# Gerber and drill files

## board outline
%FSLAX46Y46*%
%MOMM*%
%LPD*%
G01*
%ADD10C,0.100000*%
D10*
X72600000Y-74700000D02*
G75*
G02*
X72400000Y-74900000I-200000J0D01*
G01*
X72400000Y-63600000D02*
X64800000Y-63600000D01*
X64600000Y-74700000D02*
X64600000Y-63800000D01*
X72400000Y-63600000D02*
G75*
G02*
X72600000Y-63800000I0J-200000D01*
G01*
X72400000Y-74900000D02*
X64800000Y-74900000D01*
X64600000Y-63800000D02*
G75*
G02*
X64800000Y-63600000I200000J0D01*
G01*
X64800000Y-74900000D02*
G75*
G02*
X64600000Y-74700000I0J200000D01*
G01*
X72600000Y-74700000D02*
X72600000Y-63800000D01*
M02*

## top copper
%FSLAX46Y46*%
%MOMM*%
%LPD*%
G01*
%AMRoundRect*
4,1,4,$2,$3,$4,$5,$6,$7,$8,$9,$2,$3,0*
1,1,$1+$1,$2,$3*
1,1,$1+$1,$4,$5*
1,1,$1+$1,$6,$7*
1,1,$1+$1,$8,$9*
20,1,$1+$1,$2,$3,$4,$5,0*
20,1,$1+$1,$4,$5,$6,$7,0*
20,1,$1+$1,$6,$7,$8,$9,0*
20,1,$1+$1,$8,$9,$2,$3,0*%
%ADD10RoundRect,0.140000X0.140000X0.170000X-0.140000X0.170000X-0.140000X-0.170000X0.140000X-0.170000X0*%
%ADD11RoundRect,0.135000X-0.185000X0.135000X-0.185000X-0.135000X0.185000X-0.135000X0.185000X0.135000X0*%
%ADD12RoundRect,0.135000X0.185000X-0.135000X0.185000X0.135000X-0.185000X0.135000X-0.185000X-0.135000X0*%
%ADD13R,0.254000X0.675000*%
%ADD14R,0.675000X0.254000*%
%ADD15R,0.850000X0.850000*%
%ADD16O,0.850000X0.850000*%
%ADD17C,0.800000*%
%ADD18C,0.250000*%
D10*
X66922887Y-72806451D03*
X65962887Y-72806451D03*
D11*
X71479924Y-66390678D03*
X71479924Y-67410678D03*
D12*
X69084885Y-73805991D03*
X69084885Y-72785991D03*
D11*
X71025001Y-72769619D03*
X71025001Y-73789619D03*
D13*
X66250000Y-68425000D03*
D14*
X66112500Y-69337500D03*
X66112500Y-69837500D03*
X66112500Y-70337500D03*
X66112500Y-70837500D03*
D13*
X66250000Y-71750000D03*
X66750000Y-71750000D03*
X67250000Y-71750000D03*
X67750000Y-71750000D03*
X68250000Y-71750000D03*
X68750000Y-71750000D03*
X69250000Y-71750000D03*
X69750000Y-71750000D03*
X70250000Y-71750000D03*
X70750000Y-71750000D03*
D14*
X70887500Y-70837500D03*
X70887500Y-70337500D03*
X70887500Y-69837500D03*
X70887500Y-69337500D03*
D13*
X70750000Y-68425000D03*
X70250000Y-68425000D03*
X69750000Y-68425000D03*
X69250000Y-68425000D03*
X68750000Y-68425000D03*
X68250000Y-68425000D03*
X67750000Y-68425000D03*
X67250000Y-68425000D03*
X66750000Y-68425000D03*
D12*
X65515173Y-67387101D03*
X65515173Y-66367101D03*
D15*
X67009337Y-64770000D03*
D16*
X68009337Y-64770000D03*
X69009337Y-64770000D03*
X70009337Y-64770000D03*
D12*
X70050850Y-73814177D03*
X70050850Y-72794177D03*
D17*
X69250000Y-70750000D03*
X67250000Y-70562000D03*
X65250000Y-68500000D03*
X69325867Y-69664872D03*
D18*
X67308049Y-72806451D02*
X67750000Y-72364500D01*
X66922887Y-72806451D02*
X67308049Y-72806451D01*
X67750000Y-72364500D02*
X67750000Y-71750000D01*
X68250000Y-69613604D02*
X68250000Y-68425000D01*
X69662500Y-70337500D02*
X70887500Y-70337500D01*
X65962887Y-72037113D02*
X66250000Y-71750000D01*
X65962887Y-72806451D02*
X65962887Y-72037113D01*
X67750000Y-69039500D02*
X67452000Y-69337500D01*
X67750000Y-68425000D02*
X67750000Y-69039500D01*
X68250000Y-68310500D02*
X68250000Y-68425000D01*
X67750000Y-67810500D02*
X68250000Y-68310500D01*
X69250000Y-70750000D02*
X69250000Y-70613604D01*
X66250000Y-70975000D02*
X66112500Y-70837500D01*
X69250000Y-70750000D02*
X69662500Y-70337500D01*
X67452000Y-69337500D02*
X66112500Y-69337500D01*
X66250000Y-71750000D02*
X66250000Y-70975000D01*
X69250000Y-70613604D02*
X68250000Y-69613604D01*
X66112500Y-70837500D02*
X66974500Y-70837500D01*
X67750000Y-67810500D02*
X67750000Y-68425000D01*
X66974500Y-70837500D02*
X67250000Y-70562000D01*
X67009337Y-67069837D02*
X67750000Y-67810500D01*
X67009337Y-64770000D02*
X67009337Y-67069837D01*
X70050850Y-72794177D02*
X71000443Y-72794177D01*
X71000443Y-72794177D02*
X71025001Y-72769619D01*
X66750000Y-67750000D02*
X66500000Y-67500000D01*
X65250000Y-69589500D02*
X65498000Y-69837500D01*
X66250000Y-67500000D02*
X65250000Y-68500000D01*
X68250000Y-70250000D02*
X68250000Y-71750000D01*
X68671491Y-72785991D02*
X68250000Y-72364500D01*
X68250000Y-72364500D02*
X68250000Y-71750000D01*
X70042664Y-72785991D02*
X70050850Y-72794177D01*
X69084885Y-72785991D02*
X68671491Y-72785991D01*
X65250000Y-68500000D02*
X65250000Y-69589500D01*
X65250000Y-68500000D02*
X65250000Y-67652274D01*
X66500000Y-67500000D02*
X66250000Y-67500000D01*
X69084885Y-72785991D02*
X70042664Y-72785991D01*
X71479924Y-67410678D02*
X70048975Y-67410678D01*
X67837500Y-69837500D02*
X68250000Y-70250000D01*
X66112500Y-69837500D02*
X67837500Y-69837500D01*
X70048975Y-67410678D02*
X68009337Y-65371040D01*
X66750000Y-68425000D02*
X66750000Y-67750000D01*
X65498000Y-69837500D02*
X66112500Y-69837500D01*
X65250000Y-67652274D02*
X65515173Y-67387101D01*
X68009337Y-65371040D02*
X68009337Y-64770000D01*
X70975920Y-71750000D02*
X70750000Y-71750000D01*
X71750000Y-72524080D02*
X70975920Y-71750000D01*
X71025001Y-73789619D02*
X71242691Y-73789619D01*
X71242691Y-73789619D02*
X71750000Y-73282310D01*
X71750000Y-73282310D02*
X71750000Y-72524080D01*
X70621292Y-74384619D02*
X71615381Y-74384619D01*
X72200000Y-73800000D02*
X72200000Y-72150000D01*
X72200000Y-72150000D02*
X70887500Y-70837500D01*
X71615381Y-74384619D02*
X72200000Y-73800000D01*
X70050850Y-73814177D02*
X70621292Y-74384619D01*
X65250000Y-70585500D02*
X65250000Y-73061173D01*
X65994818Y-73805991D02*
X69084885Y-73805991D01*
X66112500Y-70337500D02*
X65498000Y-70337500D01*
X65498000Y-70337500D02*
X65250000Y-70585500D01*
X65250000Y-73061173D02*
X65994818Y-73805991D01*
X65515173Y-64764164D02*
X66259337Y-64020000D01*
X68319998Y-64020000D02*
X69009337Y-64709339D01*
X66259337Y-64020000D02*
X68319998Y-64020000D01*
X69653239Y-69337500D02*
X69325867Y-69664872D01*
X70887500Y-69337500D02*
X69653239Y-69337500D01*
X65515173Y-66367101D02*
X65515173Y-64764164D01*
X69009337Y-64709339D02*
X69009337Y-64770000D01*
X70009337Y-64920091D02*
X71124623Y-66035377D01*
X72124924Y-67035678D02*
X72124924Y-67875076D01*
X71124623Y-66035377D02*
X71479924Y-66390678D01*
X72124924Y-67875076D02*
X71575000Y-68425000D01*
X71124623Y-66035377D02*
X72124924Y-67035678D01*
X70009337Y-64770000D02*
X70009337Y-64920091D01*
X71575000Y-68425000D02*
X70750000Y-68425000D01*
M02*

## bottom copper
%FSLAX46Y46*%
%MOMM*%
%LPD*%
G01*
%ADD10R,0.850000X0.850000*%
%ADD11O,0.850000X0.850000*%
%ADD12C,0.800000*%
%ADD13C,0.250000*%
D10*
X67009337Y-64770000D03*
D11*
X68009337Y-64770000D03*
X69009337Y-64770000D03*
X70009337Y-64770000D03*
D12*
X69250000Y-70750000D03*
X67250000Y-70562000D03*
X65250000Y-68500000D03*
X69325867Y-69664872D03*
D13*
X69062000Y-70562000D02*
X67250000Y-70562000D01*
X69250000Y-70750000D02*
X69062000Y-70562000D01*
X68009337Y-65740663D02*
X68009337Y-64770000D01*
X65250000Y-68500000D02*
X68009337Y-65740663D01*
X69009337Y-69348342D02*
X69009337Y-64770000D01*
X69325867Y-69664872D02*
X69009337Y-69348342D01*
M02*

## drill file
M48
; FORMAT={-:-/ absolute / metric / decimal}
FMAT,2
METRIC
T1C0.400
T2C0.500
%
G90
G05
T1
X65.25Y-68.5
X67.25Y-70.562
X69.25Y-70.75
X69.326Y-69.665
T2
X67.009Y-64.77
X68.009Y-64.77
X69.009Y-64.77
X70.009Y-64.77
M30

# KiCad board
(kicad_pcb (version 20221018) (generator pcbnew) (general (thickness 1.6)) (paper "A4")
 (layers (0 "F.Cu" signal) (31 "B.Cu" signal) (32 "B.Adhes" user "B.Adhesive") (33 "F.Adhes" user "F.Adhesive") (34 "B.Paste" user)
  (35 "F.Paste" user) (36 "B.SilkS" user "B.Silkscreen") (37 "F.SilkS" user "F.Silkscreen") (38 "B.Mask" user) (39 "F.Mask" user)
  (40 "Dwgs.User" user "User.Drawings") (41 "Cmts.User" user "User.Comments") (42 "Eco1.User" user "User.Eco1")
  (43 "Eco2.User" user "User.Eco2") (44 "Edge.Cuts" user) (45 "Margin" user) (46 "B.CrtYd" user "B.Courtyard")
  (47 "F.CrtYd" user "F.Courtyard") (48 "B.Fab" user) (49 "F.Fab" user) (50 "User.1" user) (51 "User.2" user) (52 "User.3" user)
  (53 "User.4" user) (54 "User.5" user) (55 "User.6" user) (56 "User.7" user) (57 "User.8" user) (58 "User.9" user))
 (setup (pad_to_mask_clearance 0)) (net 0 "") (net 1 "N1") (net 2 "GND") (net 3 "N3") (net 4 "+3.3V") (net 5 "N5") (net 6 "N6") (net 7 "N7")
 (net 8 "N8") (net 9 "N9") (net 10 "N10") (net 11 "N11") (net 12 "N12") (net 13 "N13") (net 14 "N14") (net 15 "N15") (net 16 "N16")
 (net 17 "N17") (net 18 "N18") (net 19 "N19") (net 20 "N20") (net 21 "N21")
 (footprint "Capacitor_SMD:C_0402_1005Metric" (layer "F.Cu") (at 66.442887 72.806451 180)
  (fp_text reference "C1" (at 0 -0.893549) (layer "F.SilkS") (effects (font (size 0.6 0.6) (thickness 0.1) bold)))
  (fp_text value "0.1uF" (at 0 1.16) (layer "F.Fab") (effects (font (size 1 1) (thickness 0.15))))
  (pad "1" smd roundrect (at -0.48 0 180) (size 0.56 0.62) (layers "F.Cu" "F.Paste" "F.Mask") (roundrect_rratio 0.25) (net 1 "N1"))
  (pad "2" smd roundrect (at 0.48 0 180) (size 0.56 0.62) (layers "F.Cu" "F.Paste" "F.Mask") (roundrect_rratio 0.25) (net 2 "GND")))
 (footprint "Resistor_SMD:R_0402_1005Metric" (layer "F.Cu") (at 71.479924 66.900678 -90)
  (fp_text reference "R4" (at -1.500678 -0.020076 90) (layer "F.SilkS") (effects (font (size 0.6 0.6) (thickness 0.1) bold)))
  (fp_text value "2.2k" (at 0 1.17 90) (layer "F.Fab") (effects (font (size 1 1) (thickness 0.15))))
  (pad "1" smd roundrect (at -0.51 0 270) (size 0.54 0.64) (layers "F.Cu" "F.Paste" "F.Mask") (roundrect_rratio 0.25) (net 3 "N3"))
  (pad "2" smd roundrect (at 0.51 0 270) (size 0.54 0.64) (layers "F.Cu" "F.Paste" "F.Mask") (roundrect_rratio 0.25) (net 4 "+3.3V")))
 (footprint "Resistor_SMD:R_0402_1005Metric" (layer "F.Cu") (at 69.084885 73.295991 90)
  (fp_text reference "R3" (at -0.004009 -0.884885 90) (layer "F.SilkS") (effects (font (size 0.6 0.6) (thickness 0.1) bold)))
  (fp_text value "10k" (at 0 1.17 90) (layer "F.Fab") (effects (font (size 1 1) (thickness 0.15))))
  (pad "1" smd roundrect (at -0.51 0 90) (size 0.54 0.64) (layers "F.Cu" "F.Paste" "F.Mask") (roundrect_rratio 0.25) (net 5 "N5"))
  (pad "2" smd roundrect (at 0.51 0 90) (size 0.54 0.64) (layers "F.Cu" "F.Paste" "F.Mask") (roundrect_rratio 0.25) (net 4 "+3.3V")))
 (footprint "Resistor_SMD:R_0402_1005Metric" (layer "F.Cu") (at 71.025001 73.279619 -90)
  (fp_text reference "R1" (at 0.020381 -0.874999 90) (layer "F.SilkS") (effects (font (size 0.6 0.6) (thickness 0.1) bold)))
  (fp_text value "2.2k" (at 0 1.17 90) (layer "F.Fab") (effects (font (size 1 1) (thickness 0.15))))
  (pad "1" smd roundrect (at -0.51 0 270) (size 0.54 0.64) (layers "F.Cu" "F.Paste" "F.Mask") (roundrect_rratio 0.25) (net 4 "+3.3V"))
  (pad "2" smd roundrect (at 0.51 0 270) (size 0.54 0.64) (layers "F.Cu" "F.Paste" "F.Mask") (roundrect_rratio 0.25) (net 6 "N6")))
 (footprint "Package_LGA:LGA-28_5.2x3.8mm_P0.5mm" (layer "F.Cu") (at 68.5 70.0875)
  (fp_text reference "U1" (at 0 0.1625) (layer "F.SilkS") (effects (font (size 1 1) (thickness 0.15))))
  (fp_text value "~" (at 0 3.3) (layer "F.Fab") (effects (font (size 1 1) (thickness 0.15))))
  (pad "1" smd rect (at -2.25 -1.6625) (size 0.254 0.675) (layers "F.Cu" "F.Paste" "F.Mask") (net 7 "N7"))
  (pad "2" smd rect (at -2.3875 -0.75 90) (size 0.254 0.675) (layers "F.Cu" "F.Paste" "F.Mask") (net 2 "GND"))
  (pad "3" smd rect (at -2.3875 -0.25 90) (size 0.254 0.675) (layers "F.Cu" "F.Paste" "F.Mask") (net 4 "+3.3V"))
  (pad "4" smd rect (at -2.3875 0.25 90) (size 0.254 0.675) (layers "F.Cu" "F.Paste" "F.Mask") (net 5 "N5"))
  (pad "5" smd rect (at -2.3875 0.75 90) (size 0.254 0.675) (layers "F.Cu" "F.Paste" "F.Mask") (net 2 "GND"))
  (pad "6" smd rect (at -2.25 1.6625) (size 0.254 0.675) (layers "F.Cu" "F.Paste" "F.Mask") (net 2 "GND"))
  (pad "7" smd rect (at -1.75 1.6625) (size 0.254 0.675) (layers "F.Cu" "F.Paste" "F.Mask") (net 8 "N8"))
  (pad "8" smd rect (at -1.25 1.6625) (size 0.254 0.675) (layers "F.Cu" "F.Paste" "F.Mask") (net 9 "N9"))
  (pad "9" smd rect (at -0.75 1.6625) (size 0.254 0.675) (layers "F.Cu" "F.Paste" "F.Mask") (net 1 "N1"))
  (pad "10" smd rect (at -0.25 1.6625) (size 0.254 0.675) (layers "F.Cu" "F.Paste" "F.Mask") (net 4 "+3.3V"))
  (pad "11" smd rect (at 0.25 1.6625) (size 0.254 0.675) (layers "F.Cu" "F.Paste" "F.Mask") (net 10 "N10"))
  (pad "12" smd rect (at 0.75 1.6625) (size 0.254 0.675) (layers "F.Cu" "F.Paste" "F.Mask") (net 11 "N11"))
  (pad "13" smd rect (at 1.25 1.6625) (size 0.254 0.675) (layers "F.Cu" "F.Paste" "F.Mask") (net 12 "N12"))
  (pad "14" smd rect (at 1.75 1.6625) (size 0.254 0.675) (layers "F.Cu" "F.Paste" "F.Mask") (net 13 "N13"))
  (pad "15" smd rect (at 2.25 1.6625) (size 0.254 0.675) (layers "F.Cu" "F.Paste" "F.Mask") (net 6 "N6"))
  (pad "16" smd rect (at 2.3875 0.75 90) (size 0.254 0.675) (layers "F.Cu" "F.Paste" "F.Mask") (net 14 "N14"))
  (pad "17" smd rect (at 2.3875 0.25 90) (size 0.254 0.675) (layers "F.Cu" "F.Paste" "F.Mask") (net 2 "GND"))
  (pad "18" smd rect (at 2.3875 -0.25 90) (size 0.254 0.675) (layers "F.Cu" "F.Paste" "F.Mask") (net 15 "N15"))
  (pad "19" smd rect (at 2.3875 -0.75 90) (size 0.254 0.675) (layers "F.Cu" "F.Paste" "F.Mask") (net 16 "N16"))
  (pad "20" smd rect (at 2.25 -1.6625) (size 0.254 0.675) (layers "F.Cu" "F.Paste" "F.Mask") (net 3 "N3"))
  (pad "21" smd rect (at 1.75 -1.6625) (size 0.254 0.675) (layers "F.Cu" "F.Paste" "F.Mask") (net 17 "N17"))
  (pad "22" smd rect (at 1.25 -1.6625) (size 0.254 0.675) (layers "F.Cu" "F.Paste" "F.Mask") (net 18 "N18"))
  (pad "23" smd rect (at 0.75 -1.6625) (size 0.254 0.675) (layers "F.Cu" "F.Paste" "F.Mask") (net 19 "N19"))
  (pad "24" smd rect (at 0.25 -1.6625) (size 0.254 0.675) (layers "F.Cu" "F.Paste" "F.Mask") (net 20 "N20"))
  (pad "25" smd rect (at -0.25 -1.6625) (size 0.254 0.675) (layers "F.Cu" "F.Paste" "F.Mask") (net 2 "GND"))
  (pad "26" smd rect (at -0.75 -1.6625) (size 0.254 0.675) (layers "F.Cu" "F.Paste" "F.Mask") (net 2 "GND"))
  (pad "27" smd rect (at -1.25 -1.6625) (size 0.254 0.675) (layers "F.Cu" "F.Paste" "F.Mask") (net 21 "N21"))
  (pad "28" smd rect (at -1.75 -1.6625) (size 0.254 0.675) (layers "F.Cu" "F.Paste" "F.Mask") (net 4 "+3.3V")))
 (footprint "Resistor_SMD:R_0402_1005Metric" (layer "F.Cu") (at 65.515173 66.877101 90)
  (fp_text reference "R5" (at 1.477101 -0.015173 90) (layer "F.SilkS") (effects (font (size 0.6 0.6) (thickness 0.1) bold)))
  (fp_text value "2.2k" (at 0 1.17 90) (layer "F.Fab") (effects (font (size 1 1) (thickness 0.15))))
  (pad "1" smd roundrect (at -0.51 0 90) (size 0.54 0.64) (layers "F.Cu" "F.Paste" "F.Mask") (roundrect_rratio 0.25) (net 4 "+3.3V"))
  (pad "2" smd roundrect (at 0.51 0 90) (size 0.54 0.64) (layers "F.Cu" "F.Paste" "F.Mask") (roundrect_rratio 0.25) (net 16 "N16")))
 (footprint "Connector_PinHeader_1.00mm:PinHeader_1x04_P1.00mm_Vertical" (layer "F.Cu") (at 67.009337 64.77 90)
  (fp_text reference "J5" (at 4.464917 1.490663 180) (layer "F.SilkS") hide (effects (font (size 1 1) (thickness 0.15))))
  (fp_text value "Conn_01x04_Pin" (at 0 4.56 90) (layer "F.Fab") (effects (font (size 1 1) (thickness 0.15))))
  (pad "1" thru_hole rect (at 0 0 90) (size 0.85 0.85) (drill 0.5) (layers "*.Cu" "*.Mask") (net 2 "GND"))
  (pad "2" thru_hole oval (at 0 1 90) (size 0.85 0.85) (drill 0.5) (layers "*.Cu" "*.Mask") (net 4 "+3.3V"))
  (pad "3" thru_hole oval (at 0 2 90) (size 0.85 0.85) (drill 0.5) (layers "*.Cu" "*.Mask") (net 16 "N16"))
  (pad "4" thru_hole oval (at 0 3 90) (size 0.85 0.85) (drill 0.5) (layers "*.Cu" "*.Mask") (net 3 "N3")))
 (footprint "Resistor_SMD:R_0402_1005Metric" (layer "F.Cu") (at 70.05085 73.304177 90)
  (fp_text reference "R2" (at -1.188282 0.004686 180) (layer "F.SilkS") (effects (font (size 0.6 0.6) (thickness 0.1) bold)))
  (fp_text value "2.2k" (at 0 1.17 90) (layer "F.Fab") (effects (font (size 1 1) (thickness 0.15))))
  (pad "1" smd roundrect (at -0.51 0 90) (size 0.54 0.64) (layers "F.Cu" "F.Paste" "F.Mask") (roundrect_rratio 0.25) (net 14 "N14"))
  (pad "2" smd roundrect (at 0.51 0 90) (size 0.54 0.64) (layers "F.Cu" "F.Paste" "F.Mask") (roundrect_rratio 0.25) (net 4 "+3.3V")))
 (gr_arc (start 72.6 74.7) (mid 72.541421 74.841421) (end 72.4 74.9) (stroke (width 0.1) (type default)) (layer "Edge.Cuts"))
 (gr_line (start 72.4 63.6) (end 64.8 63.6) (stroke (width 0.1) (type default)) (layer "Edge.Cuts"))
 (gr_line (start 64.6 74.7) (end 64.6 63.8) (stroke (width 0.1) (type default)) (layer "Edge.Cuts"))
 (gr_arc (start 72.4 63.6) (mid 72.541421 63.658579) (end 72.6 63.8) (stroke (width 0.1) (type default)) (layer "Edge.Cuts"))
 (gr_line (start 72.4 74.9) (end 64.8 74.9) (stroke (width 0.1) (type default)) (layer "Edge.Cuts"))
 (gr_arc (start 64.6 63.8) (mid 64.658579 63.658579) (end 64.8 63.6) (stroke (width 0.1) (type default)) (layer "Edge.Cuts"))
 (gr_arc (start 64.8 74.9) (mid 64.658579 74.841421) (end 64.6 74.7) (stroke (width 0.1) (type default)) (layer "Edge.Cuts"))
 (gr_line (start 72.6 74.7) (end 72.6 63.8) (stroke (width 0.1) (type default)) (layer "Edge.Cuts"))
 (segment (start 67.308049 72.806451) (end 67.75 72.3645) (width 0.25) (layer "F.Cu") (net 1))
 (segment (start 66.922887 72.806451) (end 67.308049 72.806451) (width 0.25) (layer "F.Cu") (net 1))
 (segment (start 67.75 72.3645) (end 67.75 71.75) (width 0.25) (layer "F.Cu") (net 1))
 (segment (start 68.25 69.613604) (end 68.25 68.425) (width 0.25) (layer "F.Cu") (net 2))
 (segment (start 69.6625 70.3375) (end 70.8875 70.3375) (width 0.25) (layer "F.Cu") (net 2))
 (segment (start 65.962887 72.037113) (end 66.25 71.75) (width 0.25) (layer "F.Cu") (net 2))
 (segment (start 65.962887 72.806451) (end 65.962887 72.037113) (width 0.25) (layer "F.Cu") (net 2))
 (segment (start 67.75 69.0395) (end 67.452 69.3375) (width 0.25) (layer "F.Cu") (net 2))
 (segment (start 67.75 68.425) (end 67.75 69.0395) (width 0.25) (layer "F.Cu") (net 2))
 (segment (start 68.25 68.3105) (end 68.25 68.425) (width 0.25) (layer "F.Cu") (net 2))
 (segment (start 67.75 67.8105) (end 68.25 68.3105) (width 0.25) (layer "F.Cu") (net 2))
 (segment (start 69.25 70.75) (end 69.25 70.613604) (width 0.25) (layer "F.Cu") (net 2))
 (segment (start 66.25 70.975) (end 66.1125 70.8375) (width 0.25) (layer "F.Cu") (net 2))
 (segment (start 69.25 70.75) (end 69.6625 70.3375) (width 0.25) (layer "F.Cu") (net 2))
 (segment (start 67.452 69.3375) (end 66.1125 69.3375) (width 0.25) (layer "F.Cu") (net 2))
 (segment (start 66.25 71.75) (end 66.25 70.975) (width 0.25) (layer "F.Cu") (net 2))
 (segment (start 69.25 70.613604) (end 68.25 69.613604) (width 0.25) (layer "F.Cu") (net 2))
 (segment (start 66.1125 70.8375) (end 66.9745 70.8375) (width 0.25) (layer "F.Cu") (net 2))
 (segment (start 67.75 67.8105) (end 67.75 68.425) (width 0.25) (layer "F.Cu") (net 2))
 (segment (start 66.9745 70.8375) (end 67.25 70.562) (width 0.25) (layer "F.Cu") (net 2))
 (segment (start 67.009337 67.069837) (end 67.75 67.8105) (width 0.25) (layer "F.Cu") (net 2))
 (segment (start 67.009337 64.77) (end 67.009337 67.069837) (width 0.25) (layer "F.Cu") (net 2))
 (via (at 69.25 70.75) (size 0.8) (drill 0.4) (layers "F.Cu" "B.Cu") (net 2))
 (via (at 67.25 70.562) (size 0.8) (drill 0.4) (layers "F.Cu" "B.Cu") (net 2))
 (segment (start 69.062 70.562) (end 67.25 70.562) (width 0.25) (layer "B.Cu") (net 2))
 (segment (start 69.25 70.75) (end 69.062 70.562) (width 0.25) (layer "B.Cu") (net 2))
 (segment (start 70.05085 72.794177) (end 71.000443 72.794177) (width 0.25) (layer "F.Cu") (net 4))
 (segment (start 71.000443 72.794177) (end 71.025001 72.769619) (width 0.25) (layer "F.Cu") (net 4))
 (segment (start 66.75 67.75) (end 66.5 67.5) (width 0.25) (layer "F.Cu") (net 4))
 (segment (start 65.25 69.5895) (end 65.498 69.8375) (width 0.25) (layer "F.Cu") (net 4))
 (segment (start 66.25 67.5) (end 65.25 68.5) (width 0.25) (layer "F.Cu") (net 4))
 (segment (start 68.25 70.25) (end 68.25 71.75) (width 0.25) (layer "F.Cu") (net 4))
 (segment (start 68.671491 72.785991) (end 68.25 72.3645) (width 0.25) (layer "F.Cu") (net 4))
 (segment (start 68.25 72.3645) (end 68.25 71.75) (width 0.25) (layer "F.Cu") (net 4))
 (segment (start 70.042664 72.785991) (end 70.05085 72.794177) (width 0.25) (layer "F.Cu") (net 4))
 (segment (start 69.084885 72.785991) (end 68.671491 72.785991) (width 0.25) (layer "F.Cu") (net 4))
 (segment (start 65.25 68.5) (end 65.25 69.5895) (width 0.25) (layer "F.Cu") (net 4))
 (segment (start 65.25 68.5) (end 65.25 67.652274) (width 0.25) (layer "F.Cu") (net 4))
 (segment (start 66.5 67.5) (end 66.25 67.5) (width 0.25) (layer "F.Cu") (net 4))
 (segment (start 69.084885 72.785991) (end 70.042664 72.785991) (width 0.25) (layer "F.Cu") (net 4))
 (segment (start 71.479924 67.410678) (end 70.048975 67.410678) (width 0.25) (layer "F.Cu") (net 4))
 (segment (start 67.8375 69.8375) (end 68.25 70.25) (width 0.25) (layer "F.Cu") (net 4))
 (segment (start 66.1125 69.8375) (end 67.8375 69.8375) (width 0.25) (layer "F.Cu") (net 4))
 (segment (start 70.048975 67.410678) (end 68.009337 65.37104) (width 0.25) (layer "F.Cu") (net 4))
 (segment (start 66.75 68.425) (end 66.75 67.75) (width 0.25) (layer "F.Cu") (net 4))
 (segment (start 65.498 69.8375) (end 66.1125 69.8375) (width 0.25) (layer "F.Cu") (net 4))
 (segment (start 65.25 67.652274) (end 65.515173 67.387101) (width 0.25) (layer "F.Cu") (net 4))
 (segment (start 68.009337 65.37104) (end 68.009337 64.77) (width 0.25) (layer "F.Cu") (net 4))
 (via (at 65.25 68.5) (size 0.8) (drill 0.4) (layers "F.Cu" "B.Cu") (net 4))
 (segment (start 68.009337 65.740663) (end 68.009337 64.77) (width 0.25) (layer "B.Cu") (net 4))
 (segment (start 65.25 68.5) (end 68.009337 65.740663) (width 0.25) (layer "B.Cu") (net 4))
 (segment (start 70.97592 71.75) (end 70.75 71.75) (width 0.25) (layer "F.Cu") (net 6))
 (segment (start 71.75 72.52408) (end 70.97592 71.75) (width 0.25) (layer "F.Cu") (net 6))
 (segment (start 71.025001 73.789619) (end 71.242691 73.789619) (width 0.25) (layer "F.Cu") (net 6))
 (segment (start 71.242691 73.789619) (end 71.75 73.28231) (width 0.25) (layer "F.Cu") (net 6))
 (segment (start 71.75 73.28231) (end 71.75 72.52408) (width 0.25) (layer "F.Cu") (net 6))
 (segment (start 70.621292 74.384619) (end 71.615381 74.384619) (width 0.25) (layer "F.Cu") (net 14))
 (segment (start 72.2 73.8) (end 72.2 72.15) (width 0.25) (layer "F.Cu") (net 14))
 (segment (start 72.2 72.15) (end 70.8875 70.8375) (width 0.25) (layer "F.Cu") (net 14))
 (segment (start 71.615381 74.384619) (end 72.2 73.8) (width 0.25) (layer "F.Cu") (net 14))
 (segment (start 70.05085 73.814177) (end 70.621292 74.384619) (width 0.25) (layer "F.Cu") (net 14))
 (segment (start 65.25 70.5855) (end 65.25 73.061173) (width 0.25) (layer "F.Cu") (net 5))
 (segment (start 65.994818 73.805991) (end 69.084885 73.805991) (width 0.25) (layer "F.Cu") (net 5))
 (segment (start 66.1125 70.3375) (end 65.498 70.3375) (width 0.25) (layer "F.Cu") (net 5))
 (segment (start 65.498 70.3375) (end 65.25 70.5855) (width 0.25) (layer "F.Cu") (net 5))
 (segment (start 65.25 73.061173) (end 65.994818 73.805991) (width 0.25) (layer "F.Cu") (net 5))
 (segment (start 65.515173 64.764164) (end 66.259337 64.02) (width 0.25) (layer "F.Cu") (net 16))
 (segment (start 68.319998 64.02) (end 69.009337 64.709339) (width 0.25) (layer "F.Cu") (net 16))
 (segment (start 66.259337 64.02) (end 68.319998 64.02) (width 0.25) (layer "F.Cu") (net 16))
 (segment (start 69.653239 69.3375) (end 69.325867 69.664872) (width 0.25) (layer "F.Cu") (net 16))
 (segment (start 70.8875 69.3375) (end 69.653239 69.3375) (width 0.25) (layer "F.Cu") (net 16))
 (segment (start 65.515173 66.367101) (end 65.515173 64.764164) (width 0.25) (layer "F.Cu") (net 16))
 (segment (start 69.009337 64.709339) (end 69.009337 64.77) (width 0.25) (layer "F.Cu") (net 16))
 (via (at 69.325867 69.664872) (size 0.8) (drill 0.4) (layers "F.Cu" "B.Cu") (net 16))
 (segment (start 69.009337 69.348342) (end 69.009337 64.77) (width 0.25) (layer "B.Cu") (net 16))
 (segment (start 69.325867 69.664872) (end 69.009337 69.348342) (width 0.25) (layer "B.Cu") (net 16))
 (segment (start 70.009337 64.920091) (end 71.124623 66.035377) (width 0.25) (layer "F.Cu") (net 3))
 (segment (start 72.124924 67.035678) (end 72.124924 67.875076) (width 0.25) (layer "F.Cu") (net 3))
 (segment (start 71.124623 66.035377) (end 71.479924 66.390678) (width 0.25) (layer "F.Cu") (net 3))
 (segment (start 72.124924 67.875076) (end 71.575 68.425) (width 0.25) (layer "F.Cu") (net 3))
 (segment (start 71.124623 66.035377) (end 72.124924 67.035678) (width 0.25) (layer "F.Cu") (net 3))
 (segment (start 70.009337 64.77) (end 70.009337 64.920091) (width 0.25) (layer "F.Cu") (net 3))
 (segment (start 71.575 68.425) (end 70.75 68.425) (width 0.25) (layer "F.Cu") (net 3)))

